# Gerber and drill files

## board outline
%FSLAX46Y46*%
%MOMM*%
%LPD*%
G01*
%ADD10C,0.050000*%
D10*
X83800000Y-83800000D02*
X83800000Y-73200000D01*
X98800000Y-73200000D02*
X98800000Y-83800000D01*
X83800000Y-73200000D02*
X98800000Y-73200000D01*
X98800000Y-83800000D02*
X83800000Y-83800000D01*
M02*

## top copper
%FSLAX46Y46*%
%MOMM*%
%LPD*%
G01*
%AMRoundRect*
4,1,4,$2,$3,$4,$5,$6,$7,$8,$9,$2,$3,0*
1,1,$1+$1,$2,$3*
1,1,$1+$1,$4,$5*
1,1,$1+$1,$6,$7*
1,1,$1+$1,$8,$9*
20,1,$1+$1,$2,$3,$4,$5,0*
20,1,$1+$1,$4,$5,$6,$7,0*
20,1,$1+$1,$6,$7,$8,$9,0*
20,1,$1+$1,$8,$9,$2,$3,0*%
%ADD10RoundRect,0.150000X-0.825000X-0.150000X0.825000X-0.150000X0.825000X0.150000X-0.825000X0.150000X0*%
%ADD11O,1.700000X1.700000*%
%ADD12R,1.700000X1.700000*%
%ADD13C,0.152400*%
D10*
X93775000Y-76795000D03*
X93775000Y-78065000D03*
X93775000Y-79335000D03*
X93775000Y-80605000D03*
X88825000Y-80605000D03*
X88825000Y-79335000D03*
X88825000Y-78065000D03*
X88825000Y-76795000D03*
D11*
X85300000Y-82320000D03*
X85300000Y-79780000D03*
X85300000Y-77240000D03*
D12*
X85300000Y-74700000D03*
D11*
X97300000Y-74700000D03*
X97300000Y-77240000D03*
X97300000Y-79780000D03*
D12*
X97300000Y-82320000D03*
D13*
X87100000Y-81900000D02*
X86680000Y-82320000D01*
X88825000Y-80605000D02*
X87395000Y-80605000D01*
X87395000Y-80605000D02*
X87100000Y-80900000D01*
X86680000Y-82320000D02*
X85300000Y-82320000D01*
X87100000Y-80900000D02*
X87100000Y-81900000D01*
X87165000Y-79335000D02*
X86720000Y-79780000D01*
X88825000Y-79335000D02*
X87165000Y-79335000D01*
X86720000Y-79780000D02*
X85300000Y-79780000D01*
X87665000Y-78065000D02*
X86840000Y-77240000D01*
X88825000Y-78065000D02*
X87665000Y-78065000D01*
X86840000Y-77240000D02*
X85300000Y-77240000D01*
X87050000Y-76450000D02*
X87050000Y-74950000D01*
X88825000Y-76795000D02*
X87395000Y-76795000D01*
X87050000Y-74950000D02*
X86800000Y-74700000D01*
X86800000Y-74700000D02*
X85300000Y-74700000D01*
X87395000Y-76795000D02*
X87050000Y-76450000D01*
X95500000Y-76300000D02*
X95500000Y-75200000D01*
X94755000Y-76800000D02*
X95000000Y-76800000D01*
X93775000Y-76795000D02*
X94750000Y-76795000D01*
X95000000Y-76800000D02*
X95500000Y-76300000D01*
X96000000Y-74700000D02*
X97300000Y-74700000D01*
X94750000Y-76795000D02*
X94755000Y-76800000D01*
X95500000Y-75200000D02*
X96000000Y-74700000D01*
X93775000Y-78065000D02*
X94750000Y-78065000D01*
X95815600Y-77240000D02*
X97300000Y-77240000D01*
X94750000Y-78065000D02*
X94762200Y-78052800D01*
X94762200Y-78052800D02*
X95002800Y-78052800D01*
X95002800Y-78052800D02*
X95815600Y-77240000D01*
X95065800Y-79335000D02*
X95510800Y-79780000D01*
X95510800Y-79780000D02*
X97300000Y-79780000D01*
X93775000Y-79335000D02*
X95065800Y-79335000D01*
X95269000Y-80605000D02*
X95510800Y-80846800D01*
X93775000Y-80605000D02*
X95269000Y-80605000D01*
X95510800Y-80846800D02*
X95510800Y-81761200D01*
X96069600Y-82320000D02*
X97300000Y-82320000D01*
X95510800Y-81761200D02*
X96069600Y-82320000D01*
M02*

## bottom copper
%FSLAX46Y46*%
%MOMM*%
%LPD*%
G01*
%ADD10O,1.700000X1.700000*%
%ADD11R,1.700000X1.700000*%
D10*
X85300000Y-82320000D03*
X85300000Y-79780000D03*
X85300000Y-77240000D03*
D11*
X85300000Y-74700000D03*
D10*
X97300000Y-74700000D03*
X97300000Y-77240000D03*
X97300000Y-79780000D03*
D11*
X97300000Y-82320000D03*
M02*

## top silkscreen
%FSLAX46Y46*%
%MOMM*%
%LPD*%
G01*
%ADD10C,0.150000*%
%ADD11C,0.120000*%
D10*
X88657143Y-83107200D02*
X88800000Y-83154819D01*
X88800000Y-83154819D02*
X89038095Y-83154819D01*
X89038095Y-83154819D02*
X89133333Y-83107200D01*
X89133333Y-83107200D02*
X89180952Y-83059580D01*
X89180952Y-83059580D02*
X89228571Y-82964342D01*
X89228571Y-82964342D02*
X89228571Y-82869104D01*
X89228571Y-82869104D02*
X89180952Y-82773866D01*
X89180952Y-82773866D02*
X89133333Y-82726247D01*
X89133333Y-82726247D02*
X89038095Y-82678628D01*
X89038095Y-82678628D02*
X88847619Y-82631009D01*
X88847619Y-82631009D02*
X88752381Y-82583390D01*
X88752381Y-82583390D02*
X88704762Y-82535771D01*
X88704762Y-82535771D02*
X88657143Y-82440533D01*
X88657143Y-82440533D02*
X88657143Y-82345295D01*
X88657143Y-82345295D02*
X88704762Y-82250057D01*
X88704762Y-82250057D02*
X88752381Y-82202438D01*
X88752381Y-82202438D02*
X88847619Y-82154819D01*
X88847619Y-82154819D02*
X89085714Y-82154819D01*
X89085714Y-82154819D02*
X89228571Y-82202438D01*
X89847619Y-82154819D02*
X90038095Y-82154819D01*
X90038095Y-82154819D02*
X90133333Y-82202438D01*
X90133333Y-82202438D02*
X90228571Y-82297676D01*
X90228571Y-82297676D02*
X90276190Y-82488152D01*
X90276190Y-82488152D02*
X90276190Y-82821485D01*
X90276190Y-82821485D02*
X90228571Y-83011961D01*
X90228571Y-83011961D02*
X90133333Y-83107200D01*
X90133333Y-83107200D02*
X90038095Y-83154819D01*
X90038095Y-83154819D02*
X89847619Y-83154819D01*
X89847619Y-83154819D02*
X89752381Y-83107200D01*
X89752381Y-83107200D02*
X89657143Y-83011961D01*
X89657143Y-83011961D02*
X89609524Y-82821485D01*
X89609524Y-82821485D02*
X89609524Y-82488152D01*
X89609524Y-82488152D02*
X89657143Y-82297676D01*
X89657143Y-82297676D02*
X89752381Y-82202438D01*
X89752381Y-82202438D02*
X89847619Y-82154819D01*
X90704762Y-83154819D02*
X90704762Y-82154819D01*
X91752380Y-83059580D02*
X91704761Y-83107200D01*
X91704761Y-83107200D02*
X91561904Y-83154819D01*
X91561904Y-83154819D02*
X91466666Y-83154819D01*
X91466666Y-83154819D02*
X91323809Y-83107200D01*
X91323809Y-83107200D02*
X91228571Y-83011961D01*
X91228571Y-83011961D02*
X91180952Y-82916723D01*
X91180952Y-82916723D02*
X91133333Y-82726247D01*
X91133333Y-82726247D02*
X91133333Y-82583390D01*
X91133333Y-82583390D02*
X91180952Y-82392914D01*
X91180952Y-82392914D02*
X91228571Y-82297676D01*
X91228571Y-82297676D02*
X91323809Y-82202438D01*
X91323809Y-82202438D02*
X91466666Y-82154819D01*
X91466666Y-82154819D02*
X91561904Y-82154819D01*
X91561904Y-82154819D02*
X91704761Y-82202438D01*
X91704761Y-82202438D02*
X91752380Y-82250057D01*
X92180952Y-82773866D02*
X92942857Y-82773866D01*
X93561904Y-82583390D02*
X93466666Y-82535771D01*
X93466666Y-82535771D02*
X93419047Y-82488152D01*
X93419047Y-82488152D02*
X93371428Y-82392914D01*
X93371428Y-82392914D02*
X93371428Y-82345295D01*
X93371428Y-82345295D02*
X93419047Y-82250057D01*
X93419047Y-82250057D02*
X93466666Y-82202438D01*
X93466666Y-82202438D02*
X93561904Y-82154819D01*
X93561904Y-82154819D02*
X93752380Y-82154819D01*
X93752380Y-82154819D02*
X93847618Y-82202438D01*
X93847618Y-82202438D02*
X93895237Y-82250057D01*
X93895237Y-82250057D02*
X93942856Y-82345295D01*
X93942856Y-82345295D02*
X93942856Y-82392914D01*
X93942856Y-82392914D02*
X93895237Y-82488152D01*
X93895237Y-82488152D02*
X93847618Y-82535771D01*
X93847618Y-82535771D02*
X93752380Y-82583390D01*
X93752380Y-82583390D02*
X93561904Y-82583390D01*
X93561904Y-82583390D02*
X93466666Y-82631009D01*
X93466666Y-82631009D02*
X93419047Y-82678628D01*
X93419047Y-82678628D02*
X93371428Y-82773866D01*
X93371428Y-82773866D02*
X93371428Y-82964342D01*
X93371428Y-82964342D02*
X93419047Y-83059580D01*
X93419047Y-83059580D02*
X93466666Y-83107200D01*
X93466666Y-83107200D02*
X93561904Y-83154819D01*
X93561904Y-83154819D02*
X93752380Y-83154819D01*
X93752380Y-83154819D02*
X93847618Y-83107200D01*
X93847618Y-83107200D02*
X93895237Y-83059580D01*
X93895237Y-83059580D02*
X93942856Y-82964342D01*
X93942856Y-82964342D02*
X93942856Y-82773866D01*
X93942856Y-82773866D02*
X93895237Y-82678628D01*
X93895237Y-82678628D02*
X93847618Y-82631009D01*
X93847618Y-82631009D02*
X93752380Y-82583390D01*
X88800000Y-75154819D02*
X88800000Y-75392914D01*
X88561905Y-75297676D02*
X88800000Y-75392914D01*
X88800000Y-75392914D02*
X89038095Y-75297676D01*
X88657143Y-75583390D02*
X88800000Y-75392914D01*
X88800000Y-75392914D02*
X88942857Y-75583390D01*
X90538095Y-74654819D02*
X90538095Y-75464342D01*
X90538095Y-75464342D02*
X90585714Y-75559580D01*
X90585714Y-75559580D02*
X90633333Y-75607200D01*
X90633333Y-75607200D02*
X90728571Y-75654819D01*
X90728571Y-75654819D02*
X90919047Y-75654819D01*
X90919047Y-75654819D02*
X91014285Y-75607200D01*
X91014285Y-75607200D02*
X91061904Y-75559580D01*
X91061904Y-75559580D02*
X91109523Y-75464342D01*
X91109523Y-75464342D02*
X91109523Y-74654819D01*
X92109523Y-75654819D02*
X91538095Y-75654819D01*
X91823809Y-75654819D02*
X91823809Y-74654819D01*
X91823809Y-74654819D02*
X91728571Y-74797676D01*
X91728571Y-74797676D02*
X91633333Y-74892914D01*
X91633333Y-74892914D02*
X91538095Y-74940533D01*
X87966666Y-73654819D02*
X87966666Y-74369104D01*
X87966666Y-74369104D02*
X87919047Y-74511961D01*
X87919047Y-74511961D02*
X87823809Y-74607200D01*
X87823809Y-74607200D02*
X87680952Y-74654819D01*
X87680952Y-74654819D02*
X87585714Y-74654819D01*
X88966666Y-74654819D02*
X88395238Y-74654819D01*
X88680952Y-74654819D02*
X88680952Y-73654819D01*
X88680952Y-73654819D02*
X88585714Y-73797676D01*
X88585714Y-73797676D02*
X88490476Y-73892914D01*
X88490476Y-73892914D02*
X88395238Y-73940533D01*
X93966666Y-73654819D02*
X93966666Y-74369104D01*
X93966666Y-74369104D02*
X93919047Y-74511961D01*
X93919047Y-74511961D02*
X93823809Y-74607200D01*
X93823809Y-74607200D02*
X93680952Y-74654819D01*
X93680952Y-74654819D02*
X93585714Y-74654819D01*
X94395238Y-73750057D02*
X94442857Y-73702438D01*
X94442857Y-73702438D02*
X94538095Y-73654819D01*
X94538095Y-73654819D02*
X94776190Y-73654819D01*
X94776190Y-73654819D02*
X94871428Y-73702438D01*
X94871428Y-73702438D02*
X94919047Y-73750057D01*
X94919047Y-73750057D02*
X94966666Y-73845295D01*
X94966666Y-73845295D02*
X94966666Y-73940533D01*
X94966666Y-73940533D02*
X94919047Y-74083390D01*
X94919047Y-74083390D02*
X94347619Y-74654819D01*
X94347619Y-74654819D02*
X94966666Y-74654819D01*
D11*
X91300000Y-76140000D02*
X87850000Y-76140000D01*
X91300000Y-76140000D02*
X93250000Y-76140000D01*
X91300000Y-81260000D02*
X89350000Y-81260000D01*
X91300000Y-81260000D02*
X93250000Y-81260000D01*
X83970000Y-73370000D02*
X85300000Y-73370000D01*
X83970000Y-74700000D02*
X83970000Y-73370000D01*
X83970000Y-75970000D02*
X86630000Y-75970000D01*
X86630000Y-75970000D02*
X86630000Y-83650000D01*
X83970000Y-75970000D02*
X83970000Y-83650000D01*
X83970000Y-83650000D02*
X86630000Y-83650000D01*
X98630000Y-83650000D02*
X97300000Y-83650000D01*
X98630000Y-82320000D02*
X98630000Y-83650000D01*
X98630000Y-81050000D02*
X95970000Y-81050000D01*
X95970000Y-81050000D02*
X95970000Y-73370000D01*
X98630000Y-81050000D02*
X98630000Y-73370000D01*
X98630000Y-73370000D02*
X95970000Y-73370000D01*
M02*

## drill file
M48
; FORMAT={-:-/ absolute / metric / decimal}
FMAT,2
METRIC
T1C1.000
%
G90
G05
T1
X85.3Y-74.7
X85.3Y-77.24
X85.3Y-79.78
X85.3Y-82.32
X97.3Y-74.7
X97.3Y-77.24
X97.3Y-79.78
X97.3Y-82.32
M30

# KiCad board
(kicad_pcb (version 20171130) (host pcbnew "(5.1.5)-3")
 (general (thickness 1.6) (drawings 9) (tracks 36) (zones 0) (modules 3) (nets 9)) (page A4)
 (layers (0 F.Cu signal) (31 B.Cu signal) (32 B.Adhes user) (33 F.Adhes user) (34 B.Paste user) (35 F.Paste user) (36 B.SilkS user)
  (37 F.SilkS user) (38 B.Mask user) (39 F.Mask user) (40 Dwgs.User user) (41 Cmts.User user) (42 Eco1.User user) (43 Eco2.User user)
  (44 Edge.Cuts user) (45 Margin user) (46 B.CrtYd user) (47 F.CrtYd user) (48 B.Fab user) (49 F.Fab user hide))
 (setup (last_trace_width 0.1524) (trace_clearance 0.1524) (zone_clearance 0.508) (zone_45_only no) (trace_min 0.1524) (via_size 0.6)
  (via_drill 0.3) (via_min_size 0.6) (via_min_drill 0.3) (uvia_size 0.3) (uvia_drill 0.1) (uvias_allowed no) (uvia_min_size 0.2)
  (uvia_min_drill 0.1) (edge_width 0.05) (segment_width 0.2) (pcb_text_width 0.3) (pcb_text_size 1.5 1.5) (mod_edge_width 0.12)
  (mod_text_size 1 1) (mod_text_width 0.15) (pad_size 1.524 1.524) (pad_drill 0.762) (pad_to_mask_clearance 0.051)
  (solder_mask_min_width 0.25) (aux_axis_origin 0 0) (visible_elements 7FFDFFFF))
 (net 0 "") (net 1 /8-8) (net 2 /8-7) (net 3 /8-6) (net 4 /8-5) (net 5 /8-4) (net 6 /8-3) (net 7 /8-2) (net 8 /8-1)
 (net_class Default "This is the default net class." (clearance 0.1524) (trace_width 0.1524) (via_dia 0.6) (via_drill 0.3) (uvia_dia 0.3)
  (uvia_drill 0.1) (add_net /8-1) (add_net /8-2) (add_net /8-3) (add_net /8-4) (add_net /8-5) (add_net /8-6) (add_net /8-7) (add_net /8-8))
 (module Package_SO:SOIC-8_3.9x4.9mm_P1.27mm (layer F.Cu) (at 91.3 78.7)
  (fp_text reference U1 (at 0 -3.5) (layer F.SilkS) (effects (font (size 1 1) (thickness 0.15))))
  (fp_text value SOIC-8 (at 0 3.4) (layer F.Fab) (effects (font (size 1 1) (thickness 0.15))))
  (fp_line (start 0 -2.56) (end -3.45 -2.56) (layer F.SilkS) (width 0.12))
  (fp_line (start 0 -2.56) (end 1.95 -2.56) (layer F.SilkS) (width 0.12))
  (fp_line (start 0 2.56) (end -1.95 2.56) (layer F.SilkS) (width 0.12))
  (fp_line (start 0 2.56) (end 1.95 2.56) (layer F.SilkS) (width 0.12))
  (pad 8 smd roundrect (at 2.475 -1.905) (size 1.95 0.6) (layers F.Cu F.Paste F.Mask) (roundrect_rratio 0.25) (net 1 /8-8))
  (pad 7 smd roundrect (at 2.475 -0.635) (size 1.95 0.6) (layers F.Cu F.Paste F.Mask) (roundrect_rratio 0.25) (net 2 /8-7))
  (pad 6 smd roundrect (at 2.475 0.635) (size 1.95 0.6) (layers F.Cu F.Paste F.Mask) (roundrect_rratio 0.25) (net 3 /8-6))
  (pad 5 smd roundrect (at 2.475 1.905) (size 1.95 0.6) (layers F.Cu F.Paste F.Mask) (roundrect_rratio 0.25) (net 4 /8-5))
  (pad 4 smd roundrect (at -2.475 1.905) (size 1.95 0.6) (layers F.Cu F.Paste F.Mask) (roundrect_rratio 0.25) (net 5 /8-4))
  (pad 3 smd roundrect (at -2.475 0.635) (size 1.95 0.6) (layers F.Cu F.Paste F.Mask) (roundrect_rratio 0.25) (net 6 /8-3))
  (pad 2 smd roundrect (at -2.475 -0.635) (size 1.95 0.6) (layers F.Cu F.Paste F.Mask) (roundrect_rratio 0.25) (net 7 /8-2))
  (pad 1 smd roundrect (at -2.475 -1.905) (size 1.95 0.6) (layers F.Cu F.Paste F.Mask) (roundrect_rratio 0.25) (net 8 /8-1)))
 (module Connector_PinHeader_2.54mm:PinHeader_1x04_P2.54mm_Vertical (layer F.Cu) (at 85.3 74.7)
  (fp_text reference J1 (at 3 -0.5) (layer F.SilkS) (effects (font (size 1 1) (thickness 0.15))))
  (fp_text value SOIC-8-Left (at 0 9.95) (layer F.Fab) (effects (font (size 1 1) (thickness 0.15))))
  (fp_line (start -1.33 -1.33) (end 0 -1.33) (layer F.SilkS) (width 0.12))
  (fp_line (start -1.33 0) (end -1.33 -1.33) (layer F.SilkS) (width 0.12))
  (fp_line (start -1.33 1.27) (end 1.33 1.27) (layer F.SilkS) (width 0.12))
  (fp_line (start 1.33 1.27) (end 1.33 8.95) (layer F.SilkS) (width 0.12))
  (fp_line (start -1.33 1.27) (end -1.33 8.95) (layer F.SilkS) (width 0.12))
  (fp_line (start -1.33 8.95) (end 1.33 8.95) (layer F.SilkS) (width 0.12))
  (pad 4 thru_hole oval (at 0 7.62) (size 1.7 1.7) (drill 1) (layers *.Cu *.Mask) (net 5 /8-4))
  (pad 3 thru_hole oval (at 0 5.08) (size 1.7 1.7) (drill 1) (layers *.Cu *.Mask) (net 6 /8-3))
  (pad 2 thru_hole oval (at 0 2.54) (size 1.7 1.7) (drill 1) (layers *.Cu *.Mask) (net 7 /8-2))
  (pad 1 thru_hole rect (at 0 0) (size 1.7 1.7) (drill 1) (layers *.Cu *.Mask) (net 8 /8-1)))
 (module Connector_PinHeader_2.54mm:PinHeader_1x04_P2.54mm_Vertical (layer F.Cu) (at 97.3 82.32 180)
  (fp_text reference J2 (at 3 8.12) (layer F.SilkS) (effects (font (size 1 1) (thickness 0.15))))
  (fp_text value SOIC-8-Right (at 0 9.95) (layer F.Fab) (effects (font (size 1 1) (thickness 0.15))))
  (fp_line (start -1.33 -1.33) (end 0 -1.33) (layer F.SilkS) (width 0.12))
  (fp_line (start -1.33 0) (end -1.33 -1.33) (layer F.SilkS) (width 0.12))
  (fp_line (start -1.33 1.27) (end 1.33 1.27) (layer F.SilkS) (width 0.12))
  (fp_line (start 1.33 1.27) (end 1.33 8.95) (layer F.SilkS) (width 0.12))
  (fp_line (start -1.33 1.27) (end -1.33 8.95) (layer F.SilkS) (width 0.12))
  (fp_line (start -1.33 8.95) (end 1.33 8.95) (layer F.SilkS) (width 0.12))
  (pad 4 thru_hole oval (at 0 7.62 180) (size 1.7 1.7) (drill 1) (layers *.Cu *.Mask) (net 1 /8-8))
  (pad 3 thru_hole oval (at 0 5.08 180) (size 1.7 1.7) (drill 1) (layers *.Cu *.Mask) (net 2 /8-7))
  (pad 2 thru_hole oval (at 0 2.54 180) (size 1.7 1.7) (drill 1) (layers *.Cu *.Mask) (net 3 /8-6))
  (pad 1 thru_hole rect (at 0 0 180) (size 1.7 1.7) (drill 1) (layers *.Cu *.Mask) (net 4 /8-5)))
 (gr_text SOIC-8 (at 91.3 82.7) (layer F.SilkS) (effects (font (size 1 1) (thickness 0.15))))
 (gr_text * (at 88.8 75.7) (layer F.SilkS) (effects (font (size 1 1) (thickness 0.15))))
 (gr_line (start 83.8 83.8) (end 83.8 73.2) (layer Edge.Cuts) (width 0.05))
 (gr_line (start 98.8 73.2) (end 98.8 83.8) (layer Edge.Cuts) (width 0.05))
 (gr_line (start 83.8 73.2) (end 98.8 73.2) (layer Edge.Cuts) (width 0.05))
 (gr_line (start 98.8 83.8) (end 83.8 83.8) (layer Edge.Cuts) (width 0.05))
 (segment (start 87.1 81.9) (end 86.68 82.32) (width 0.1524) (layer F.Cu) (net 5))
 (segment (start 88.825 80.605) (end 87.395 80.605) (width 0.1524) (layer F.Cu) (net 5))
 (segment (start 87.395 80.605) (end 87.1 80.9) (width 0.1524) (layer F.Cu) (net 5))
 (segment (start 86.68 82.32) (end 85.3 82.32) (width 0.1524) (layer F.Cu) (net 5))
 (segment (start 87.1 80.9) (end 87.1 81.9) (width 0.1524) (layer F.Cu) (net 5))
 (segment (start 87.165 79.335) (end 86.72 79.78) (width 0.1524) (layer F.Cu) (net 6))
 (segment (start 88.825 79.335) (end 87.165 79.335) (width 0.1524) (layer F.Cu) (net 6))
 (segment (start 86.72 79.78) (end 85.3 79.78) (width 0.1524) (layer F.Cu) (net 6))
 (segment (start 87.665 78.065) (end 86.84 77.24) (width 0.1524) (layer F.Cu) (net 7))
 (segment (start 88.825 78.065) (end 87.665 78.065) (width 0.1524) (layer F.Cu) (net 7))
 (segment (start 86.84 77.24) (end 85.3 77.24) (width 0.1524) (layer F.Cu) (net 7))
 (segment (start 87.05 76.45) (end 87.05 74.95) (width 0.1524) (layer F.Cu) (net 8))
 (segment (start 88.825 76.795) (end 87.395 76.795) (width 0.1524) (layer F.Cu) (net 8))
 (segment (start 87.05 74.95) (end 86.8 74.7) (width 0.1524) (layer F.Cu) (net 8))
 (segment (start 86.8 74.7) (end 85.3 74.7) (width 0.1524) (layer F.Cu) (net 8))
 (segment (start 87.395 76.795) (end 87.05 76.45) (width 0.1524) (layer F.Cu) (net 8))
 (segment (start 95.5 76.3) (end 95.5 75.2) (width 0.1524) (layer F.Cu) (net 1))
 (segment (start 94.755 76.8) (end 95 76.8) (width 0.1524) (layer F.Cu) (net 1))
 (segment (start 93.775 76.795) (end 94.75 76.795) (width 0.1524) (layer F.Cu) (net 1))
 (segment (start 95 76.8) (end 95.5 76.3) (width 0.1524) (layer F.Cu) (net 1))
 (segment (start 96 74.7) (end 97.3 74.7) (width 0.1524) (layer F.Cu) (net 1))
 (segment (start 94.75 76.795) (end 94.755 76.8) (width 0.1524) (layer F.Cu) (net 1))
 (segment (start 95.5 75.2) (end 96 74.7) (width 0.1524) (layer F.Cu) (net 1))
 (segment (start 93.775 78.065) (end 94.75 78.065) (width 0.1524) (layer F.Cu) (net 2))
 (segment (start 95.8156 77.24) (end 97.3 77.24) (width 0.1524) (layer F.Cu) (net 2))
 (segment (start 94.75 78.065) (end 94.7622 78.0528) (width 0.1524) (layer F.Cu) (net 2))
 (segment (start 94.7622 78.0528) (end 95.0028 78.0528) (width 0.1524) (layer F.Cu) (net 2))
 (segment (start 95.0028 78.0528) (end 95.8156 77.24) (width 0.1524) (layer F.Cu) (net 2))
 (segment (start 95.0658 79.335) (end 95.5108 79.78) (width 0.1524) (layer F.Cu) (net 3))
 (segment (start 95.5108 79.78) (end 97.3 79.78) (width 0.1524) (layer F.Cu) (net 3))
 (segment (start 93.775 79.335) (end 95.0658 79.335) (width 0.1524) (layer F.Cu) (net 3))
 (segment (start 95.269 80.605) (end 95.5108 80.8468) (width 0.1524) (layer F.Cu) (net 4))
 (segment (start 93.775 80.605) (end 95.269 80.605) (width 0.1524) (layer F.Cu) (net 4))
 (segment (start 95.5108 80.8468) (end 95.5108 81.7612) (width 0.1524) (layer F.Cu) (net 4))
 (segment (start 96.0696 82.32) (end 97.3 82.32) (width 0.1524) (layer F.Cu) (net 4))
 (segment (start 95.5108 81.7612) (end 96.0696 82.32) (width 0.1524) (layer F.Cu) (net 4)))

